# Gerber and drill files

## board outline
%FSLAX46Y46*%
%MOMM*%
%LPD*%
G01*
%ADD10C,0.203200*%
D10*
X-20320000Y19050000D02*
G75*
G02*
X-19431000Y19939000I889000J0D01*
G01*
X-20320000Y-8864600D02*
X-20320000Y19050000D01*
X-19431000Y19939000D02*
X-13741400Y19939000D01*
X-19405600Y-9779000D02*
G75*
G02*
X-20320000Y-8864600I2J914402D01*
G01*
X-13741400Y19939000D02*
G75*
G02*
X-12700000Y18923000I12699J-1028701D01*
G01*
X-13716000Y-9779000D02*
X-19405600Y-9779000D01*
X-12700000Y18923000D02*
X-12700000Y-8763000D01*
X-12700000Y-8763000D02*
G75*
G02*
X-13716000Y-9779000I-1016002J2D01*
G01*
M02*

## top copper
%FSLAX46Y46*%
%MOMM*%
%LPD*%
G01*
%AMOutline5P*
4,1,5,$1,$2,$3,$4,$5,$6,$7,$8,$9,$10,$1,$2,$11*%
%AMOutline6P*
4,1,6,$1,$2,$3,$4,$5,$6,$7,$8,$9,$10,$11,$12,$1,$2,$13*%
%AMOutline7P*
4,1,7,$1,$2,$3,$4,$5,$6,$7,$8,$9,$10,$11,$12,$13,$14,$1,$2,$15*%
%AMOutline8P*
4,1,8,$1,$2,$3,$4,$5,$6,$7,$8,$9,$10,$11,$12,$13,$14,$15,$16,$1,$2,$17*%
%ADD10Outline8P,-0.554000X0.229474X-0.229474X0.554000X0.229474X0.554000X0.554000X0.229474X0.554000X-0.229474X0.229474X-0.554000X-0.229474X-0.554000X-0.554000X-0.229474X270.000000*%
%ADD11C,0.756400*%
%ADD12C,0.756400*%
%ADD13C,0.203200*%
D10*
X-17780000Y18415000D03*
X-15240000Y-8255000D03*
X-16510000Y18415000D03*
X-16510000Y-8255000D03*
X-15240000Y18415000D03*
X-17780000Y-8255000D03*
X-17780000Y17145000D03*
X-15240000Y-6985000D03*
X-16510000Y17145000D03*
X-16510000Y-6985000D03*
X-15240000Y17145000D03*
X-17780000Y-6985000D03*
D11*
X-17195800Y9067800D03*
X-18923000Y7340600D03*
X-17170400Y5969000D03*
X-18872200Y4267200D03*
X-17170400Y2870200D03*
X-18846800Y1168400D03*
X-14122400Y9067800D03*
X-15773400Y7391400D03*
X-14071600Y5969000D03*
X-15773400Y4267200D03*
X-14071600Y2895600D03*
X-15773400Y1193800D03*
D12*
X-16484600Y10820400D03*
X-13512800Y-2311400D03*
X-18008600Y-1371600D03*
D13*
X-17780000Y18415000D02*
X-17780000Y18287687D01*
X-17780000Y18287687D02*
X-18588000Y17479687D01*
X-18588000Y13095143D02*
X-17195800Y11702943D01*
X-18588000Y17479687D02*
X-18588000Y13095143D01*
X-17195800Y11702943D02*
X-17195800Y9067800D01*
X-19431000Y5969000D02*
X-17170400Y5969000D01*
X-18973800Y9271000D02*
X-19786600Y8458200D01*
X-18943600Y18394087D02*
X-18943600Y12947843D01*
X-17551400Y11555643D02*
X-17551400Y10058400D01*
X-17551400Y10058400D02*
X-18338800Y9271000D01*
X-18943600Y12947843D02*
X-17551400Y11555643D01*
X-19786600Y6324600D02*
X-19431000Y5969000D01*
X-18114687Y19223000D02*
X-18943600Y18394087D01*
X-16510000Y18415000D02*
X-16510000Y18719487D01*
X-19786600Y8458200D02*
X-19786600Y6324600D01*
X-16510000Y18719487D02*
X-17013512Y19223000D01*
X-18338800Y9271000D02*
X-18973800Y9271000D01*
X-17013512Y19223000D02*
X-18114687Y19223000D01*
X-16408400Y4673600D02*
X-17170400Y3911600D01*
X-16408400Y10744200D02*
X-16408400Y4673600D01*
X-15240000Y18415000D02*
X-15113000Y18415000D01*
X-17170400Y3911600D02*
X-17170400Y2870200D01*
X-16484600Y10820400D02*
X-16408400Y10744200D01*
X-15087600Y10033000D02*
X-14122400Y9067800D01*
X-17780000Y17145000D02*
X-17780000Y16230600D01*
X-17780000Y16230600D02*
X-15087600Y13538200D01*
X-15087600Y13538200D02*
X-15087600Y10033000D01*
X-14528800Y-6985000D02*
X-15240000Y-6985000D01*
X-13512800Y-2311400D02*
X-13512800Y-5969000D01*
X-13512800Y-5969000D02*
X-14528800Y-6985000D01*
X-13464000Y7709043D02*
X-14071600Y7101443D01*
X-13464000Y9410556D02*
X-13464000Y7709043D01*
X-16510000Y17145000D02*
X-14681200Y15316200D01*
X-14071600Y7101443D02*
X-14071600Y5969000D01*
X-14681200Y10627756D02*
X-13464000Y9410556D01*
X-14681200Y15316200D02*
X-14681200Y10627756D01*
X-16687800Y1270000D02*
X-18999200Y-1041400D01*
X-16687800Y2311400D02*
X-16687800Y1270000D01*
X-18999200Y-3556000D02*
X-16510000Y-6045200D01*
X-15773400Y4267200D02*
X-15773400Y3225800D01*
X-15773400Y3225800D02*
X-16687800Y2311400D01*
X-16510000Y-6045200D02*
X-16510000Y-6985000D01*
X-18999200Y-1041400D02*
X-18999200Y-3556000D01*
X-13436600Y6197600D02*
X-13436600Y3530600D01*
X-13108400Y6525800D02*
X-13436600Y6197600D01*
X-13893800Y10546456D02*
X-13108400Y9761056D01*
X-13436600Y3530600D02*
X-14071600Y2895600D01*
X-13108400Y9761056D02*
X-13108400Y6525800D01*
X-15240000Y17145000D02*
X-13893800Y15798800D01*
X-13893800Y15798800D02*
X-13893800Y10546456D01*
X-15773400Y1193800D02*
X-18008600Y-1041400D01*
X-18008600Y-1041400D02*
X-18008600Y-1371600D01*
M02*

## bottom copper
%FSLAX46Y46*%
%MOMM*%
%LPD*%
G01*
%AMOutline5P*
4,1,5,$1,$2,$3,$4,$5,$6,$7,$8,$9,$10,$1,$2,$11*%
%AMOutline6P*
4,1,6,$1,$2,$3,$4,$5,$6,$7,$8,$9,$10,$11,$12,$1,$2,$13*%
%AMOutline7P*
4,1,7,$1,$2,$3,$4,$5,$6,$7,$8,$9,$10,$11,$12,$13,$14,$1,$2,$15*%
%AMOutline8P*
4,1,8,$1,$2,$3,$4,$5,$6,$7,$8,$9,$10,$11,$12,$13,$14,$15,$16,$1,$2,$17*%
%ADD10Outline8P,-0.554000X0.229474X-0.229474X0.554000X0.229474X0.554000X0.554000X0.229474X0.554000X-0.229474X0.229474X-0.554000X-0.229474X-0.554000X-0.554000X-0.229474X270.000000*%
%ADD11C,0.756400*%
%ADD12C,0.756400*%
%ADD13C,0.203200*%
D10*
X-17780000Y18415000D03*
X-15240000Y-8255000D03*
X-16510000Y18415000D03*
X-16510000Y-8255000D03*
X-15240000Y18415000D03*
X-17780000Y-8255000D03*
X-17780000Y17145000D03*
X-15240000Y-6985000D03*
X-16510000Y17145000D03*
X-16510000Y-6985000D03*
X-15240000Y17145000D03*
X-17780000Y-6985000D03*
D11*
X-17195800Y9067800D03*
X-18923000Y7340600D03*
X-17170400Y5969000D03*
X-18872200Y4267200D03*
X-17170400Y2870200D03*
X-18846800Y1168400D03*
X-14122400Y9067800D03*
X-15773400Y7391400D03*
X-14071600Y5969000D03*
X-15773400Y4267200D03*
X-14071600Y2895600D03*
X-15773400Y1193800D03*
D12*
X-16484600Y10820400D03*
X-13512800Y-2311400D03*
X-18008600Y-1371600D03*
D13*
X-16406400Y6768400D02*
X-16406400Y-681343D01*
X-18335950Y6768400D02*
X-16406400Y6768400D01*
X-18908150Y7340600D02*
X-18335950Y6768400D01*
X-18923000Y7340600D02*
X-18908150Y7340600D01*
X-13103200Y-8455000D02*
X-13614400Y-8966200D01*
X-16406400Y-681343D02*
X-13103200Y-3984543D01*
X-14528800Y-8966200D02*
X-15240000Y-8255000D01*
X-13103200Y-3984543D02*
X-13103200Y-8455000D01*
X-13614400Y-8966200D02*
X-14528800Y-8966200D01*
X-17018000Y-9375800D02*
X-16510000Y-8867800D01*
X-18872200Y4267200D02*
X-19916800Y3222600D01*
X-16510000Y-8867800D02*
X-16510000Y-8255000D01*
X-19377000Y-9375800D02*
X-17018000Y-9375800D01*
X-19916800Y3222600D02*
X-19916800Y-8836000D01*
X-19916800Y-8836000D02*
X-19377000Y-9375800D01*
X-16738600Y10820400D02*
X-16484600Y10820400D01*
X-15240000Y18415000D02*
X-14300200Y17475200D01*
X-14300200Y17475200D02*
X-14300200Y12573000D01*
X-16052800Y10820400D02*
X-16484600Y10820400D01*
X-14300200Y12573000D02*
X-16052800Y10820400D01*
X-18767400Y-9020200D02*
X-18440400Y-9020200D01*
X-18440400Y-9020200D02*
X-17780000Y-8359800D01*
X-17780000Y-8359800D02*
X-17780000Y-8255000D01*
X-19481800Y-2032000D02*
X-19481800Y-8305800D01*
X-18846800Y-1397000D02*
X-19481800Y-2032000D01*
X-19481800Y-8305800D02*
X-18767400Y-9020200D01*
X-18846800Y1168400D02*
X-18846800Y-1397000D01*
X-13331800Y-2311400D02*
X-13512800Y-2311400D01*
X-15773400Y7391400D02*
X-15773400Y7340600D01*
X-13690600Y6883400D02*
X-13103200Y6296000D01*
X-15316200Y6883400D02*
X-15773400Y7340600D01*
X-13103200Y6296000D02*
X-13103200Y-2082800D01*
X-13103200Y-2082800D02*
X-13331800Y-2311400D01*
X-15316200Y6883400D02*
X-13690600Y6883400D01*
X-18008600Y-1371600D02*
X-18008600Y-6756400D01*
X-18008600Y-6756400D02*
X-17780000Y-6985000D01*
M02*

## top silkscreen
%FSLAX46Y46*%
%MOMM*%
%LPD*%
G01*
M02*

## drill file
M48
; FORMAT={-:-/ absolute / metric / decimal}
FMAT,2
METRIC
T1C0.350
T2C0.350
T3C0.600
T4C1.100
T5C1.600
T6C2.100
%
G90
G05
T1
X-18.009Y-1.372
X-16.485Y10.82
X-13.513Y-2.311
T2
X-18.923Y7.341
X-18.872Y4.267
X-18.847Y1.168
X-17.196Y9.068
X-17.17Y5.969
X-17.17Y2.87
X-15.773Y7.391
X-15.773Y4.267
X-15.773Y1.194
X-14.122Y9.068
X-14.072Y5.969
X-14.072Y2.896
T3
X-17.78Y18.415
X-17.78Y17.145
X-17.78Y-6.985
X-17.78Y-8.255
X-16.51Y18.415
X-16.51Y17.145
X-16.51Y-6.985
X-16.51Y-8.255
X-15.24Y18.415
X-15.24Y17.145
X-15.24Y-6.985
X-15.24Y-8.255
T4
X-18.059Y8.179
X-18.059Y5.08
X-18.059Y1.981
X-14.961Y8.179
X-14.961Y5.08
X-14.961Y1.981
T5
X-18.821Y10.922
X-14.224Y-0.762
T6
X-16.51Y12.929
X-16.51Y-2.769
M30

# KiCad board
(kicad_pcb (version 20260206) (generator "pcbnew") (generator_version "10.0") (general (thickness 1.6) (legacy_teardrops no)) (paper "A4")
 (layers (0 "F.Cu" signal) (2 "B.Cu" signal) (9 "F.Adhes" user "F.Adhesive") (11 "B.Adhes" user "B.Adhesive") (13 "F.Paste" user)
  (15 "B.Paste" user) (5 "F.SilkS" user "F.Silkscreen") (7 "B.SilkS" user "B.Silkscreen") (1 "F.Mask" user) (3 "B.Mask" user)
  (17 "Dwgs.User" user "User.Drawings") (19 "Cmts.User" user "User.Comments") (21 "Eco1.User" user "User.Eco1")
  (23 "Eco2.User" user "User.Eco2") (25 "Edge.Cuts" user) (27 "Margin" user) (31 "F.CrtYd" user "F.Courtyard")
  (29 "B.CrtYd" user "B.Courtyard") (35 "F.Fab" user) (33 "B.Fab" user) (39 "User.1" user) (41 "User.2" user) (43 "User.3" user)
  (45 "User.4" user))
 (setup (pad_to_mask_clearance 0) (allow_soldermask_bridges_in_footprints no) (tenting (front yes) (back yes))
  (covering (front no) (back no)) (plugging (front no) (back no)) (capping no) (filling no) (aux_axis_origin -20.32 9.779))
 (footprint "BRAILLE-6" (layer "F.Cu") (at -16.51 -5.08)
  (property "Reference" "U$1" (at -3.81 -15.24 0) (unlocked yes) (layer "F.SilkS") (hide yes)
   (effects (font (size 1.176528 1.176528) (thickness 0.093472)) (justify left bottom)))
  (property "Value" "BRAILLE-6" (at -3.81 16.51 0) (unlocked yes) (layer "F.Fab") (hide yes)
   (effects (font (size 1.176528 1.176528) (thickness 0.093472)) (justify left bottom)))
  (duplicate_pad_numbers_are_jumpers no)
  (pad "P$1" thru_hole roundrect (at -1.27 -13.335 270) (size 1.108 1.108) (drill 0.6) (layers "*.Cu" "*.Mask") (remove_unused_layers no)
   (roundrect_rratio 0.25) (chamfer_ratio 0.2928932188) (chamfer top_left top_right bottom_left bottom_right) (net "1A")
   (solder_mask_margin 0.025) (thermal_bridge_angle 0))
  (pad "P$2" thru_hole roundrect (at 1.27 13.335 270) (size 1.108 1.108) (drill 0.6) (layers "*.Cu" "*.Mask") (remove_unused_layers no)
   (roundrect_rratio 0.25) (chamfer_ratio 0.2928932188) (chamfer top_left top_right bottom_left bottom_right) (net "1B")
   (solder_mask_margin 0.025) (thermal_bridge_angle 0))
  (pad "P$3" thru_hole roundrect (at 0 -13.335 270) (size 1.108 1.108) (drill 0.6) (layers "*.Cu" "*.Mask") (remove_unused_layers no)
   (roundrect_rratio 0.25) (chamfer_ratio 0.2928932188) (chamfer top_left top_right bottom_left bottom_right) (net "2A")
   (solder_mask_margin 0.025) (thermal_bridge_angle 0))
  (pad "P$4" thru_hole roundrect (at 0 13.335 270) (size 1.108 1.108) (drill 0.6) (layers "*.Cu" "*.Mask") (remove_unused_layers no)
   (roundrect_rratio 0.25) (chamfer_ratio 0.2928932188) (chamfer top_left top_right bottom_left bottom_right) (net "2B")
   (solder_mask_margin 0.025) (thermal_bridge_angle 0))
  (pad "P$5" thru_hole roundrect (at 1.27 -13.335 270) (size 1.108 1.108) (drill 0.6) (layers "*.Cu" "*.Mask") (remove_unused_layers no)
   (roundrect_rratio 0.25) (chamfer_ratio 0.2928932188) (chamfer top_left top_right bottom_left bottom_right) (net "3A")
   (solder_mask_margin 0.025) (thermal_bridge_angle 0))
  (pad "P$6" thru_hole roundrect (at -1.27 13.335 270) (size 1.108 1.108) (drill 0.6) (layers "*.Cu" "*.Mask") (remove_unused_layers no)
   (roundrect_rratio 0.25) (chamfer_ratio 0.2928932188) (chamfer top_left top_right bottom_left bottom_right) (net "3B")
   (solder_mask_margin 0.025) (thermal_bridge_angle 0))
  (pad "P$7" thru_hole roundrect (at -1.27 -12.065 270) (size 1.108 1.108) (drill 0.6) (layers "*.Cu" "*.Mask") (remove_unused_layers no)
   (roundrect_rratio 0.25) (chamfer_ratio 0.2928932188) (chamfer top_left top_right bottom_left bottom_right) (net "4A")
   (solder_mask_margin 0.025) (thermal_bridge_angle 0))
  (pad "P$8" thru_hole roundrect (at 1.27 12.065 270) (size 1.108 1.108) (drill 0.6) (layers "*.Cu" "*.Mask") (remove_unused_layers no)
   (roundrect_rratio 0.25) (chamfer_ratio 0.2928932188) (chamfer top_left top_right bottom_left bottom_right) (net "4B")
   (solder_mask_margin 0.025) (thermal_bridge_angle 0))
  (pad "P$9" thru_hole roundrect (at 0 -12.065 270) (size 1.108 1.108) (drill 0.6) (layers "*.Cu" "*.Mask") (remove_unused_layers no)
   (roundrect_rratio 0.25) (chamfer_ratio 0.2928932188) (chamfer top_left top_right bottom_left bottom_right) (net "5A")
   (solder_mask_margin 0.025) (thermal_bridge_angle 0))
  (pad "P$10" thru_hole roundrect (at 0 12.065 270) (size 1.108 1.108) (drill 0.6) (layers "*.Cu" "*.Mask") (remove_unused_layers no)
   (roundrect_rratio 0.25) (chamfer_ratio 0.2928932188) (chamfer top_left top_right bottom_left bottom_right) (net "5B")
   (solder_mask_margin 0.025) (thermal_bridge_angle 0))
  (pad "P$11" thru_hole roundrect (at 1.27 -12.065 270) (size 1.108 1.108) (drill 0.6) (layers "*.Cu" "*.Mask") (remove_unused_layers no)
   (roundrect_rratio 0.25) (chamfer_ratio 0.2928932188) (chamfer top_left top_right bottom_left bottom_right) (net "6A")
   (solder_mask_margin 0.025) (thermal_bridge_angle 0))
  (pad "P$12" thru_hole roundrect (at -1.27 12.065 270) (size 1.108 1.108) (drill 0.6) (layers "*.Cu" "*.Mask") (remove_unused_layers no)
   (roundrect_rratio 0.25) (chamfer_ratio 0.2928932188) (chamfer top_left top_right bottom_left bottom_right) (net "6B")
   (solder_mask_margin 0.025) (thermal_bridge_angle 0)))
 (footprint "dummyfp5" (layer "F.Cu") (at -14.9606 -1.9812)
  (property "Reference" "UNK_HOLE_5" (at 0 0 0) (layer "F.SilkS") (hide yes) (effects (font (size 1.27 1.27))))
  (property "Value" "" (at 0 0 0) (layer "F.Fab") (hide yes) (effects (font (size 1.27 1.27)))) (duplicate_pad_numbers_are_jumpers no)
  (pad "" np_thru_hole circle (at 0 0) (size 1.1 1.1) (drill 1.1) (layers "*.Cu" "*.Mask")))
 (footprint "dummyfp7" (layer "F.Cu") (at -16.51 2.7686)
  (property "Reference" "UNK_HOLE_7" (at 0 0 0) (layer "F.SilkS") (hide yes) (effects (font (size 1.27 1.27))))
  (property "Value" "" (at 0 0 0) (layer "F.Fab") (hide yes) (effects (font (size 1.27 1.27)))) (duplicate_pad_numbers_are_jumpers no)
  (pad "" np_thru_hole circle (at 0 0) (size 2.1 2.1) (drill 2.1) (layers "*.Cu" "*.Mask")))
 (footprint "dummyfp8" (layer "F.Cu") (at -18.8214 -10.922)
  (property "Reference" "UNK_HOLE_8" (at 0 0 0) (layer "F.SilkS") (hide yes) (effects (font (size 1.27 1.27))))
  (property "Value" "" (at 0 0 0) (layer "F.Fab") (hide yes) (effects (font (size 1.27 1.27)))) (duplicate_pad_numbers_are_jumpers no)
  (pad "" np_thru_hole circle (at 0 0) (size 1.6 1.6) (drill 1.6) (layers "*.Cu" "*.Mask")))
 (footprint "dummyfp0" (layer "F.Cu") (at -18.0594 -8.1788)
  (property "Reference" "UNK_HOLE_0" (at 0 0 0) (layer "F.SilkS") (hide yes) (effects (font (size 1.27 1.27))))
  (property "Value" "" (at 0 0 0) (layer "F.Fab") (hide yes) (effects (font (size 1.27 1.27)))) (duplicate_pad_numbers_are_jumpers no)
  (pad "" np_thru_hole circle (at 0 0) (size 1.1 1.1) (drill 1.1) (layers "*.Cu" "*.Mask")))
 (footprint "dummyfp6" (layer "F.Cu") (at -16.51 -12.9286)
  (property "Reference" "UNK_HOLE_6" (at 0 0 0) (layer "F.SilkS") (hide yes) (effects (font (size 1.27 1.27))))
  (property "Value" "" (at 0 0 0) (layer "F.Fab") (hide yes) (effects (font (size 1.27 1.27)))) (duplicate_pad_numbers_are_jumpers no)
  (pad "" np_thru_hole circle (at 0 0) (size 2.1 2.1) (drill 2.1) (layers "*.Cu" "*.Mask")))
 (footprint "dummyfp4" (layer "F.Cu") (at -18.0594 -1.9812)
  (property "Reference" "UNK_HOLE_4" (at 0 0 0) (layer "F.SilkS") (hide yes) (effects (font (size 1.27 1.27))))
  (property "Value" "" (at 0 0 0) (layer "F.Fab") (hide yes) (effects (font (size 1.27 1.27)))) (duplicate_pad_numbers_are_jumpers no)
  (pad "" np_thru_hole circle (at 0 0) (size 1.1 1.1) (drill 1.1) (layers "*.Cu" "*.Mask")))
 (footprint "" (layer "F.Cu") (at 0 0)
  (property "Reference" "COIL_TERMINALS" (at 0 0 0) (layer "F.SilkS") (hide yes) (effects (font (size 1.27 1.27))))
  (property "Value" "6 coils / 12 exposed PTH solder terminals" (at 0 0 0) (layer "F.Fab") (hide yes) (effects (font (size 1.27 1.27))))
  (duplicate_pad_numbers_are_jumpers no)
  (pad "1A" thru_hole circle (at -17.1958 -9.0678) (size 0.7564 0.7564) (drill 0.35) (layers "*.Cu" "*.Mask") (remove_unused_layers no)
   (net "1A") (solder_mask_margin 0.025))
  (pad "1B" thru_hole circle (at -18.923 -7.3406) (size 0.7564 0.7564) (drill 0.35) (layers "*.Cu" "*.Mask") (remove_unused_layers no)
   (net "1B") (solder_mask_margin 0.025))
  (pad "2A" thru_hole circle (at -17.1704 -5.969) (size 0.7564 0.7564) (drill 0.35) (layers "*.Cu" "*.Mask") (remove_unused_layers no)
   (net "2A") (solder_mask_margin 0.025))
  (pad "2B" thru_hole circle (at -18.8722 -4.2672) (size 0.7564 0.7564) (drill 0.35) (layers "*.Cu" "*.Mask") (remove_unused_layers no)
   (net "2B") (solder_mask_margin 0.025))
  (pad "3A" thru_hole circle (at -17.1704 -2.8702) (size 0.7564 0.7564) (drill 0.35) (layers "*.Cu" "*.Mask") (remove_unused_layers no)
   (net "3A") (solder_mask_margin 0.025))
  (pad "3B" thru_hole circle (at -18.8468 -1.1684) (size 0.7564 0.7564) (drill 0.35) (layers "*.Cu" "*.Mask") (remove_unused_layers no)
   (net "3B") (solder_mask_margin 0.025))
  (pad "4A" thru_hole circle (at -14.1224 -9.0678) (size 0.7564 0.7564) (drill 0.35) (layers "*.Cu" "*.Mask") (remove_unused_layers no)
   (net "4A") (solder_mask_margin 0.025))
  (pad "4B" thru_hole circle (at -15.7734 -7.3914) (size 0.7564 0.7564) (drill 0.35) (layers "*.Cu" "*.Mask") (remove_unused_layers no)
   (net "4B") (solder_mask_margin 0.025))
  (pad "5A" thru_hole circle (at -14.0716 -5.969) (size 0.7564 0.7564) (drill 0.35) (layers "*.Cu" "*.Mask") (remove_unused_layers no)
   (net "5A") (solder_mask_margin 0.025))
  (pad "5B" thru_hole circle (at -15.7734 -4.2672) (size 0.7564 0.7564) (drill 0.35) (layers "*.Cu" "*.Mask") (remove_unused_layers no)
   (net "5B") (solder_mask_margin 0.025))
  (pad "6A" thru_hole circle (at -14.0716 -2.8956) (size 0.7564 0.7564) (drill 0.35) (layers "*.Cu" "*.Mask") (remove_unused_layers no)
   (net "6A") (solder_mask_margin 0.025))
  (pad "6B" thru_hole circle (at -15.7734 -1.1938) (size 0.7564 0.7564) (drill 0.35) (layers "*.Cu" "*.Mask") (remove_unused_layers no)
   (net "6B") (solder_mask_margin 0.025)))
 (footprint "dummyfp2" (layer "F.Cu") (at -18.0594 -5.08)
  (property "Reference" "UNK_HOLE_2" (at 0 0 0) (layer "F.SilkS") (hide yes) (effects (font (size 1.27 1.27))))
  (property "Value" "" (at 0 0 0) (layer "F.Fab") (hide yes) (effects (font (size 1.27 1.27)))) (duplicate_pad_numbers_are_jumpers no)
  (pad "" np_thru_hole circle (at 0 0) (size 1.1 1.1) (drill 1.1) (layers "*.Cu" "*.Mask")))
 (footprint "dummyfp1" (layer "F.Cu") (at -14.9606 -8.1788)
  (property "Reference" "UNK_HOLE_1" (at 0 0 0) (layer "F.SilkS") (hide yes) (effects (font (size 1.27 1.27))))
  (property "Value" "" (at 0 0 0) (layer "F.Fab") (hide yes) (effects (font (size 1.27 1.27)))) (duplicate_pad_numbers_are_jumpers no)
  (pad "" np_thru_hole circle (at 0 0) (size 1.1 1.1) (drill 1.1) (layers "*.Cu" "*.Mask")))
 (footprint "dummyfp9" (layer "F.Cu") (at -14.224 0.762)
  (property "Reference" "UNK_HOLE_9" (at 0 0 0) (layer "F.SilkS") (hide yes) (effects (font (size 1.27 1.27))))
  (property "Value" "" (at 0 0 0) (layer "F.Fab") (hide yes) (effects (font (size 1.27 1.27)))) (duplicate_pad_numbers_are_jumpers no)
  (pad "" np_thru_hole circle (at 0 0) (size 1.6 1.6) (drill 1.6) (layers "*.Cu" "*.Mask")))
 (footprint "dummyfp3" (layer "F.Cu") (at -14.9606 -5.08)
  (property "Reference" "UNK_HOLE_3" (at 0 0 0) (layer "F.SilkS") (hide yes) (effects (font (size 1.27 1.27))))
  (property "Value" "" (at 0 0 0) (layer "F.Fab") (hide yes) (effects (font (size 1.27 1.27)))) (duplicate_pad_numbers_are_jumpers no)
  (pad "" np_thru_hole circle (at 0 0) (size 1.1 1.1) (drill 1.1) (layers "*.Cu" "*.Mask")))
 (gr_arc (start -20.32 -19.05) (mid -20.059618 -19.678618) (end -19.431 -19.939) (stroke (width 0.2032) (type solid)) (layer "Edge.Cuts"))
 (gr_line (start -20.32 8.8646) (end -20.32 -19.05) (stroke (width 0.2032) (type solid)) (layer "Edge.Cuts"))
 (gr_line (start -19.431 -19.939) (end -13.7414 -19.939) (stroke (width 0.2032) (type solid)) (layer "Edge.Cuts"))
 (gr_arc (start -19.4056 9.779) (mid -20.052178 9.511178) (end -20.32 8.8646) (stroke (width 0.2032) (type solid)) (layer "Edge.Cuts"))
 (gr_arc (start -13.7414 -19.939) (mid -13.01028 -19.646681) (end -12.7 -18.923) (stroke (width 0.2032) (type solid)) (layer "Edge.Cuts"))
 (gr_line (start -13.716 9.779) (end -19.4056 9.779) (stroke (width 0.2032) (type solid)) (layer "Edge.Cuts"))
 (gr_line (start -12.7 -18.923) (end -12.7 8.763) (stroke (width 0.2032) (type solid)) (layer "Edge.Cuts"))
 (gr_arc (start -12.7 8.763) (mid -12.99758 9.48142) (end -13.716 9.779) (stroke (width 0.2032) (type solid)) (layer "Edge.Cuts"))
 (segment (start -17.78 -18.415) (end -17.78 -18.287687) (width 0.2032) (layer "F.Cu") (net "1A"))
 (segment (start -17.78 -18.287687) (end -18.588 -17.479687) (width 0.2032) (layer "F.Cu") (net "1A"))
 (segment (start -18.588 -13.095143) (end -17.1958 -11.702943) (width 0.2032) (layer "F.Cu") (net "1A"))
 (segment (start -18.588 -17.479687) (end -18.588 -13.095143) (width 0.2032) (layer "F.Cu") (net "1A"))
 (segment (start -17.1958 -11.702943) (end -17.1958 -9.0678) (width 0.2032) (layer "F.Cu") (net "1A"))
 (segment (start -16.4064 -6.7684) (end -16.4064 0.681343) (width 0.2032) (layer "B.Cu") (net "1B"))
 (segment (start -18.33595 -6.7684) (end -16.4064 -6.7684) (width 0.2032) (layer "B.Cu") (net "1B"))
 (segment (start -18.90815 -7.3406) (end -18.33595 -6.7684) (width 0.2032) (layer "B.Cu") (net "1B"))
 (segment (start -18.923 -7.3406) (end -18.90815 -7.3406) (width 0.2032) (layer "B.Cu") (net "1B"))
 (segment (start -13.1032 8.455) (end -13.6144 8.9662) (width 0.2032) (layer "B.Cu") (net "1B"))
 (segment (start -16.4064 0.681343) (end -13.1032 3.984543) (width 0.2032) (layer "B.Cu") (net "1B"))
 (segment (start -14.5288 8.9662) (end -15.24 8.255) (width 0.2032) (layer "B.Cu") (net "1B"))
 (segment (start -13.1032 3.984543) (end -13.1032 8.455) (width 0.2032) (layer "B.Cu") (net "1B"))
 (segment (start -13.6144 8.9662) (end -14.5288 8.9662) (width 0.2032) (layer "B.Cu") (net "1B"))
 (segment (start -19.431 -5.969) (end -17.1704 -5.969) (width 0.2032) (layer "F.Cu") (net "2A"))
 (segment (start -18.9738 -9.271) (end -19.7866 -8.4582) (width 0.2032) (layer "F.Cu") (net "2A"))
 (segment (start -18.9436 -18.394087) (end -18.9436 -12.947843) (width 0.2032) (layer "F.Cu") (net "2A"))
 (segment (start -17.5514 -11.555643) (end -17.5514 -10.0584) (width 0.2032) (layer "F.Cu") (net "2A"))
 (segment (start -17.5514 -10.0584) (end -18.3388 -9.271) (width 0.2032) (layer "F.Cu") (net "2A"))
 (segment (start -18.9436 -12.947843) (end -17.5514 -11.555643) (width 0.2032) (layer "F.Cu") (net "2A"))
 (segment (start -19.7866 -6.3246) (end -19.431 -5.969) (width 0.2032) (layer "F.Cu") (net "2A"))
 (segment (start -18.114687 -19.223) (end -18.9436 -18.394087) (width 0.2032) (layer "F.Cu") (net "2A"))
 (segment (start -16.51 -18.415) (end -16.51 -18.719487) (width 0.2032) (layer "F.Cu") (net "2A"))
 (segment (start -19.7866 -8.4582) (end -19.7866 -6.3246) (width 0.2032) (layer "F.Cu") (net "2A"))
 (segment (start -16.51 -18.719487) (end -17.013512 -19.223) (width 0.2032) (layer "F.Cu") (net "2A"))
 (segment (start -18.3388 -9.271) (end -18.9738 -9.271) (width 0.2032) (layer "F.Cu") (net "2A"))
 (segment (start -17.013512 -19.223) (end -18.114687 -19.223) (width 0.2032) (layer "F.Cu") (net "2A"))
 (segment (start -17.018 9.3758) (end -16.51 8.8678) (width 0.2032) (layer "B.Cu") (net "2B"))
 (segment (start -18.8722 -4.2672) (end -19.9168 -3.2226) (width 0.2032) (layer "B.Cu") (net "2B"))
 (segment (start -16.51 8.8678) (end -16.51 8.255) (width 0.2032) (layer "B.Cu") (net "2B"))
 (segment (start -19.377 9.3758) (end -17.018 9.3758) (width 0.2032) (layer "B.Cu") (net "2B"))
 (segment (start -19.9168 -3.2226) (end -19.9168 8.836) (width 0.2032) (layer "B.Cu") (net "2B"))
 (segment (start -19.9168 8.836) (end -19.377 9.3758) (width 0.2032) (layer "B.Cu") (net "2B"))
 (segment (start -16.4084 -4.6736) (end -17.1704 -3.9116) (width 0.2032) (layer "F.Cu") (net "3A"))
 (segment (start -16.4084 -10.7442) (end -16.4084 -4.6736) (width 0.2032) (layer "F.Cu") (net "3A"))
 (segment (start -15.24 -18.415) (end -15.113 -18.415) (width 0.2032) (layer "F.Cu") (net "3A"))
 (segment (start -17.1704 -3.9116) (end -17.1704 -2.8702) (width 0.2032) (layer "F.Cu") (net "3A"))
 (segment (start -16.4846 -10.8204) (end -16.4084 -10.7442) (width 0.2032) (layer "F.Cu") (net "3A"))
 (via (at -16.4846 -10.8204) (size 0.7564) (drill 0.35) (layers "F.Cu" "B.Cu") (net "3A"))
 (segment (start -16.7386 -10.8204) (end -16.4846 -10.8204) (width 0.2032) (layer "B.Cu") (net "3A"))
 (segment (start -15.24 -18.415) (end -14.3002 -17.4752) (width 0.2032) (layer "B.Cu") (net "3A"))
 (segment (start -14.3002 -17.4752) (end -14.3002 -12.573) (width 0.2032) (layer "B.Cu") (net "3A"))
 (segment (start -16.0528 -10.8204) (end -16.4846 -10.8204) (width 0.2032) (layer "B.Cu") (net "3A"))
 (segment (start -14.3002 -12.573) (end -16.0528 -10.8204) (width 0.2032) (layer "B.Cu") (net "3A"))
 (segment (start -18.7674 9.0202) (end -18.4404 9.0202) (width 0.2032) (layer "B.Cu") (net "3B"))
 (segment (start -18.4404 9.0202) (end -17.78 8.3598) (width 0.2032) (layer "B.Cu") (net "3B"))
 (segment (start -17.78 8.3598) (end -17.78 8.255) (width 0.2032) (layer "B.Cu") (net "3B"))
 (segment (start -19.4818 2.032) (end -19.4818 8.3058) (width 0.2032) (layer "B.Cu") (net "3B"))
 (segment (start -18.8468 1.397) (end -19.4818 2.032) (width 0.2032) (layer "B.Cu") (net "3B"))
 (segment (start -19.4818 8.3058) (end -18.7674 9.0202) (width 0.2032) (layer "B.Cu") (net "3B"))
 (segment (start -18.8468 -1.1684) (end -18.8468 1.397) (width 0.2032) (layer "B.Cu") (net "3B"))
 (segment (start -15.0876 -10.033) (end -14.1224 -9.0678) (width 0.2032) (layer "F.Cu") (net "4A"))
 (segment (start -17.78 -17.145) (end -17.78 -16.2306) (width 0.2032) (layer "F.Cu") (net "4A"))
 (segment (start -17.78 -16.2306) (end -15.0876 -13.5382) (width 0.2032) (layer "F.Cu") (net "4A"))
 (segment (start -15.0876 -13.5382) (end -15.0876 -10.033) (width 0.2032) (layer "F.Cu") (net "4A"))
 (segment (start -14.5288 6.985) (end -15.24 6.985) (width 0.2032) (layer "F.Cu") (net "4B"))
 (segment (start -13.5128 2.3114) (end -13.5128 5.969) (width 0.2032) (layer "F.Cu") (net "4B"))
 (segment (start -13.5128 5.969) (end -14.5288 6.985) (width 0.2032) (layer "F.Cu") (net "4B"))
 (via (at -13.5128 2.3114) (size 0.7564) (drill 0.35) (layers "F.Cu" "B.Cu") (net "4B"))
 (segment (start -13.3318 2.3114) (end -13.5128 2.3114) (width 0.2032) (layer "B.Cu") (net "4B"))
 (segment (start -15.7734 -7.3914) (end -15.7734 -7.3406) (width 0.2032) (layer "B.Cu") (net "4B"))
 (segment (start -13.6906 -6.8834) (end -13.1032 -6.296) (width 0.2032) (layer "B.Cu") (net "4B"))
 (segment (start -15.3162 -6.8834) (end -15.7734 -7.3406) (width 0.2032) (layer "B.Cu") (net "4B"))
 (segment (start -13.1032 -6.296) (end -13.1032 2.0828) (width 0.2032) (layer "B.Cu") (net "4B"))
 (segment (start -13.1032 2.0828) (end -13.3318 2.3114) (width 0.2032) (layer "B.Cu") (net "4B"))
 (segment (start -15.3162 -6.8834) (end -13.6906 -6.8834) (width 0.2032) (layer "B.Cu") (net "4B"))
 (segment (start -13.464 -7.709043) (end -14.0716 -7.101443) (width 0.2032) (layer "F.Cu") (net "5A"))
 (segment (start -13.464 -9.410556) (end -13.464 -7.709043) (width 0.2032) (layer "F.Cu") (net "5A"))
 (segment (start -16.51 -17.145) (end -14.6812 -15.3162) (width 0.2032) (layer "F.Cu") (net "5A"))
 (segment (start -14.0716 -7.101443) (end -14.0716 -5.969) (width 0.2032) (layer "F.Cu") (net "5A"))
 (segment (start -14.6812 -10.627756) (end -13.464 -9.410556) (width 0.2032) (layer "F.Cu") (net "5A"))
 (segment (start -14.6812 -15.3162) (end -14.6812 -10.627756) (width 0.2032) (layer "F.Cu") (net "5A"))
 (segment (start -16.6878 -1.27) (end -18.9992 1.0414) (width 0.2032) (layer "F.Cu") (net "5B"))
 (segment (start -16.6878 -2.3114) (end -16.6878 -1.27) (width 0.2032) (layer "F.Cu") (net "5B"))
 (segment (start -18.9992 3.556) (end -16.51 6.0452) (width 0.2032) (layer "F.Cu") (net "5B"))
 (segment (start -15.7734 -4.2672) (end -15.7734 -3.2258) (width 0.2032) (layer "F.Cu") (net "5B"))
 (segment (start -15.7734 -3.2258) (end -16.6878 -2.3114) (width 0.2032) (layer "F.Cu") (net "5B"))
 (segment (start -16.51 6.0452) (end -16.51 6.985) (width 0.2032) (layer "F.Cu") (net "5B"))
 (segment (start -18.9992 1.0414) (end -18.9992 3.556) (width 0.2032) (layer "F.Cu") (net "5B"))
 (segment (start -13.4366 -6.1976) (end -13.4366 -3.5306) (width 0.2032) (layer "F.Cu") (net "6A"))
 (segment (start -13.1084 -6.5258) (end -13.4366 -6.1976) (width 0.2032) (layer "F.Cu") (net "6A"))
 (segment (start -13.8938 -10.546456) (end -13.1084 -9.761056) (width 0.2032) (layer "F.Cu") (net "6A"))
 (segment (start -13.4366 -3.5306) (end -14.0716 -2.8956) (width 0.2032) (layer "F.Cu") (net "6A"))
 (segment (start -13.1084 -9.761056) (end -13.1084 -6.5258) (width 0.2032) (layer "F.Cu") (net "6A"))
 (segment (start -15.24 -17.145) (end -13.8938 -15.7988) (width 0.2032) (layer "F.Cu") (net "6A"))
 (segment (start -13.8938 -15.7988) (end -13.8938 -10.546456) (width 0.2032) (layer "F.Cu") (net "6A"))
 (segment (start -15.7734 -1.1938) (end -18.0086 1.0414) (width 0.2032) (layer "F.Cu") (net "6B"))
 (segment (start -18.0086 1.0414) (end -18.0086 1.3716) (width 0.2032) (layer "F.Cu") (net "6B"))
 (via (at -18.0086 1.3716) (size 0.7564) (drill 0.35) (layers "F.Cu" "B.Cu") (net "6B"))
 (segment (start -18.0086 1.3716) (end -18.0086 6.7564) (width 0.2032) (layer "B.Cu") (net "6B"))
 (segment (start -18.0086 6.7564) (end -17.78 6.985) (width 0.2032) (layer "B.Cu") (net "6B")))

